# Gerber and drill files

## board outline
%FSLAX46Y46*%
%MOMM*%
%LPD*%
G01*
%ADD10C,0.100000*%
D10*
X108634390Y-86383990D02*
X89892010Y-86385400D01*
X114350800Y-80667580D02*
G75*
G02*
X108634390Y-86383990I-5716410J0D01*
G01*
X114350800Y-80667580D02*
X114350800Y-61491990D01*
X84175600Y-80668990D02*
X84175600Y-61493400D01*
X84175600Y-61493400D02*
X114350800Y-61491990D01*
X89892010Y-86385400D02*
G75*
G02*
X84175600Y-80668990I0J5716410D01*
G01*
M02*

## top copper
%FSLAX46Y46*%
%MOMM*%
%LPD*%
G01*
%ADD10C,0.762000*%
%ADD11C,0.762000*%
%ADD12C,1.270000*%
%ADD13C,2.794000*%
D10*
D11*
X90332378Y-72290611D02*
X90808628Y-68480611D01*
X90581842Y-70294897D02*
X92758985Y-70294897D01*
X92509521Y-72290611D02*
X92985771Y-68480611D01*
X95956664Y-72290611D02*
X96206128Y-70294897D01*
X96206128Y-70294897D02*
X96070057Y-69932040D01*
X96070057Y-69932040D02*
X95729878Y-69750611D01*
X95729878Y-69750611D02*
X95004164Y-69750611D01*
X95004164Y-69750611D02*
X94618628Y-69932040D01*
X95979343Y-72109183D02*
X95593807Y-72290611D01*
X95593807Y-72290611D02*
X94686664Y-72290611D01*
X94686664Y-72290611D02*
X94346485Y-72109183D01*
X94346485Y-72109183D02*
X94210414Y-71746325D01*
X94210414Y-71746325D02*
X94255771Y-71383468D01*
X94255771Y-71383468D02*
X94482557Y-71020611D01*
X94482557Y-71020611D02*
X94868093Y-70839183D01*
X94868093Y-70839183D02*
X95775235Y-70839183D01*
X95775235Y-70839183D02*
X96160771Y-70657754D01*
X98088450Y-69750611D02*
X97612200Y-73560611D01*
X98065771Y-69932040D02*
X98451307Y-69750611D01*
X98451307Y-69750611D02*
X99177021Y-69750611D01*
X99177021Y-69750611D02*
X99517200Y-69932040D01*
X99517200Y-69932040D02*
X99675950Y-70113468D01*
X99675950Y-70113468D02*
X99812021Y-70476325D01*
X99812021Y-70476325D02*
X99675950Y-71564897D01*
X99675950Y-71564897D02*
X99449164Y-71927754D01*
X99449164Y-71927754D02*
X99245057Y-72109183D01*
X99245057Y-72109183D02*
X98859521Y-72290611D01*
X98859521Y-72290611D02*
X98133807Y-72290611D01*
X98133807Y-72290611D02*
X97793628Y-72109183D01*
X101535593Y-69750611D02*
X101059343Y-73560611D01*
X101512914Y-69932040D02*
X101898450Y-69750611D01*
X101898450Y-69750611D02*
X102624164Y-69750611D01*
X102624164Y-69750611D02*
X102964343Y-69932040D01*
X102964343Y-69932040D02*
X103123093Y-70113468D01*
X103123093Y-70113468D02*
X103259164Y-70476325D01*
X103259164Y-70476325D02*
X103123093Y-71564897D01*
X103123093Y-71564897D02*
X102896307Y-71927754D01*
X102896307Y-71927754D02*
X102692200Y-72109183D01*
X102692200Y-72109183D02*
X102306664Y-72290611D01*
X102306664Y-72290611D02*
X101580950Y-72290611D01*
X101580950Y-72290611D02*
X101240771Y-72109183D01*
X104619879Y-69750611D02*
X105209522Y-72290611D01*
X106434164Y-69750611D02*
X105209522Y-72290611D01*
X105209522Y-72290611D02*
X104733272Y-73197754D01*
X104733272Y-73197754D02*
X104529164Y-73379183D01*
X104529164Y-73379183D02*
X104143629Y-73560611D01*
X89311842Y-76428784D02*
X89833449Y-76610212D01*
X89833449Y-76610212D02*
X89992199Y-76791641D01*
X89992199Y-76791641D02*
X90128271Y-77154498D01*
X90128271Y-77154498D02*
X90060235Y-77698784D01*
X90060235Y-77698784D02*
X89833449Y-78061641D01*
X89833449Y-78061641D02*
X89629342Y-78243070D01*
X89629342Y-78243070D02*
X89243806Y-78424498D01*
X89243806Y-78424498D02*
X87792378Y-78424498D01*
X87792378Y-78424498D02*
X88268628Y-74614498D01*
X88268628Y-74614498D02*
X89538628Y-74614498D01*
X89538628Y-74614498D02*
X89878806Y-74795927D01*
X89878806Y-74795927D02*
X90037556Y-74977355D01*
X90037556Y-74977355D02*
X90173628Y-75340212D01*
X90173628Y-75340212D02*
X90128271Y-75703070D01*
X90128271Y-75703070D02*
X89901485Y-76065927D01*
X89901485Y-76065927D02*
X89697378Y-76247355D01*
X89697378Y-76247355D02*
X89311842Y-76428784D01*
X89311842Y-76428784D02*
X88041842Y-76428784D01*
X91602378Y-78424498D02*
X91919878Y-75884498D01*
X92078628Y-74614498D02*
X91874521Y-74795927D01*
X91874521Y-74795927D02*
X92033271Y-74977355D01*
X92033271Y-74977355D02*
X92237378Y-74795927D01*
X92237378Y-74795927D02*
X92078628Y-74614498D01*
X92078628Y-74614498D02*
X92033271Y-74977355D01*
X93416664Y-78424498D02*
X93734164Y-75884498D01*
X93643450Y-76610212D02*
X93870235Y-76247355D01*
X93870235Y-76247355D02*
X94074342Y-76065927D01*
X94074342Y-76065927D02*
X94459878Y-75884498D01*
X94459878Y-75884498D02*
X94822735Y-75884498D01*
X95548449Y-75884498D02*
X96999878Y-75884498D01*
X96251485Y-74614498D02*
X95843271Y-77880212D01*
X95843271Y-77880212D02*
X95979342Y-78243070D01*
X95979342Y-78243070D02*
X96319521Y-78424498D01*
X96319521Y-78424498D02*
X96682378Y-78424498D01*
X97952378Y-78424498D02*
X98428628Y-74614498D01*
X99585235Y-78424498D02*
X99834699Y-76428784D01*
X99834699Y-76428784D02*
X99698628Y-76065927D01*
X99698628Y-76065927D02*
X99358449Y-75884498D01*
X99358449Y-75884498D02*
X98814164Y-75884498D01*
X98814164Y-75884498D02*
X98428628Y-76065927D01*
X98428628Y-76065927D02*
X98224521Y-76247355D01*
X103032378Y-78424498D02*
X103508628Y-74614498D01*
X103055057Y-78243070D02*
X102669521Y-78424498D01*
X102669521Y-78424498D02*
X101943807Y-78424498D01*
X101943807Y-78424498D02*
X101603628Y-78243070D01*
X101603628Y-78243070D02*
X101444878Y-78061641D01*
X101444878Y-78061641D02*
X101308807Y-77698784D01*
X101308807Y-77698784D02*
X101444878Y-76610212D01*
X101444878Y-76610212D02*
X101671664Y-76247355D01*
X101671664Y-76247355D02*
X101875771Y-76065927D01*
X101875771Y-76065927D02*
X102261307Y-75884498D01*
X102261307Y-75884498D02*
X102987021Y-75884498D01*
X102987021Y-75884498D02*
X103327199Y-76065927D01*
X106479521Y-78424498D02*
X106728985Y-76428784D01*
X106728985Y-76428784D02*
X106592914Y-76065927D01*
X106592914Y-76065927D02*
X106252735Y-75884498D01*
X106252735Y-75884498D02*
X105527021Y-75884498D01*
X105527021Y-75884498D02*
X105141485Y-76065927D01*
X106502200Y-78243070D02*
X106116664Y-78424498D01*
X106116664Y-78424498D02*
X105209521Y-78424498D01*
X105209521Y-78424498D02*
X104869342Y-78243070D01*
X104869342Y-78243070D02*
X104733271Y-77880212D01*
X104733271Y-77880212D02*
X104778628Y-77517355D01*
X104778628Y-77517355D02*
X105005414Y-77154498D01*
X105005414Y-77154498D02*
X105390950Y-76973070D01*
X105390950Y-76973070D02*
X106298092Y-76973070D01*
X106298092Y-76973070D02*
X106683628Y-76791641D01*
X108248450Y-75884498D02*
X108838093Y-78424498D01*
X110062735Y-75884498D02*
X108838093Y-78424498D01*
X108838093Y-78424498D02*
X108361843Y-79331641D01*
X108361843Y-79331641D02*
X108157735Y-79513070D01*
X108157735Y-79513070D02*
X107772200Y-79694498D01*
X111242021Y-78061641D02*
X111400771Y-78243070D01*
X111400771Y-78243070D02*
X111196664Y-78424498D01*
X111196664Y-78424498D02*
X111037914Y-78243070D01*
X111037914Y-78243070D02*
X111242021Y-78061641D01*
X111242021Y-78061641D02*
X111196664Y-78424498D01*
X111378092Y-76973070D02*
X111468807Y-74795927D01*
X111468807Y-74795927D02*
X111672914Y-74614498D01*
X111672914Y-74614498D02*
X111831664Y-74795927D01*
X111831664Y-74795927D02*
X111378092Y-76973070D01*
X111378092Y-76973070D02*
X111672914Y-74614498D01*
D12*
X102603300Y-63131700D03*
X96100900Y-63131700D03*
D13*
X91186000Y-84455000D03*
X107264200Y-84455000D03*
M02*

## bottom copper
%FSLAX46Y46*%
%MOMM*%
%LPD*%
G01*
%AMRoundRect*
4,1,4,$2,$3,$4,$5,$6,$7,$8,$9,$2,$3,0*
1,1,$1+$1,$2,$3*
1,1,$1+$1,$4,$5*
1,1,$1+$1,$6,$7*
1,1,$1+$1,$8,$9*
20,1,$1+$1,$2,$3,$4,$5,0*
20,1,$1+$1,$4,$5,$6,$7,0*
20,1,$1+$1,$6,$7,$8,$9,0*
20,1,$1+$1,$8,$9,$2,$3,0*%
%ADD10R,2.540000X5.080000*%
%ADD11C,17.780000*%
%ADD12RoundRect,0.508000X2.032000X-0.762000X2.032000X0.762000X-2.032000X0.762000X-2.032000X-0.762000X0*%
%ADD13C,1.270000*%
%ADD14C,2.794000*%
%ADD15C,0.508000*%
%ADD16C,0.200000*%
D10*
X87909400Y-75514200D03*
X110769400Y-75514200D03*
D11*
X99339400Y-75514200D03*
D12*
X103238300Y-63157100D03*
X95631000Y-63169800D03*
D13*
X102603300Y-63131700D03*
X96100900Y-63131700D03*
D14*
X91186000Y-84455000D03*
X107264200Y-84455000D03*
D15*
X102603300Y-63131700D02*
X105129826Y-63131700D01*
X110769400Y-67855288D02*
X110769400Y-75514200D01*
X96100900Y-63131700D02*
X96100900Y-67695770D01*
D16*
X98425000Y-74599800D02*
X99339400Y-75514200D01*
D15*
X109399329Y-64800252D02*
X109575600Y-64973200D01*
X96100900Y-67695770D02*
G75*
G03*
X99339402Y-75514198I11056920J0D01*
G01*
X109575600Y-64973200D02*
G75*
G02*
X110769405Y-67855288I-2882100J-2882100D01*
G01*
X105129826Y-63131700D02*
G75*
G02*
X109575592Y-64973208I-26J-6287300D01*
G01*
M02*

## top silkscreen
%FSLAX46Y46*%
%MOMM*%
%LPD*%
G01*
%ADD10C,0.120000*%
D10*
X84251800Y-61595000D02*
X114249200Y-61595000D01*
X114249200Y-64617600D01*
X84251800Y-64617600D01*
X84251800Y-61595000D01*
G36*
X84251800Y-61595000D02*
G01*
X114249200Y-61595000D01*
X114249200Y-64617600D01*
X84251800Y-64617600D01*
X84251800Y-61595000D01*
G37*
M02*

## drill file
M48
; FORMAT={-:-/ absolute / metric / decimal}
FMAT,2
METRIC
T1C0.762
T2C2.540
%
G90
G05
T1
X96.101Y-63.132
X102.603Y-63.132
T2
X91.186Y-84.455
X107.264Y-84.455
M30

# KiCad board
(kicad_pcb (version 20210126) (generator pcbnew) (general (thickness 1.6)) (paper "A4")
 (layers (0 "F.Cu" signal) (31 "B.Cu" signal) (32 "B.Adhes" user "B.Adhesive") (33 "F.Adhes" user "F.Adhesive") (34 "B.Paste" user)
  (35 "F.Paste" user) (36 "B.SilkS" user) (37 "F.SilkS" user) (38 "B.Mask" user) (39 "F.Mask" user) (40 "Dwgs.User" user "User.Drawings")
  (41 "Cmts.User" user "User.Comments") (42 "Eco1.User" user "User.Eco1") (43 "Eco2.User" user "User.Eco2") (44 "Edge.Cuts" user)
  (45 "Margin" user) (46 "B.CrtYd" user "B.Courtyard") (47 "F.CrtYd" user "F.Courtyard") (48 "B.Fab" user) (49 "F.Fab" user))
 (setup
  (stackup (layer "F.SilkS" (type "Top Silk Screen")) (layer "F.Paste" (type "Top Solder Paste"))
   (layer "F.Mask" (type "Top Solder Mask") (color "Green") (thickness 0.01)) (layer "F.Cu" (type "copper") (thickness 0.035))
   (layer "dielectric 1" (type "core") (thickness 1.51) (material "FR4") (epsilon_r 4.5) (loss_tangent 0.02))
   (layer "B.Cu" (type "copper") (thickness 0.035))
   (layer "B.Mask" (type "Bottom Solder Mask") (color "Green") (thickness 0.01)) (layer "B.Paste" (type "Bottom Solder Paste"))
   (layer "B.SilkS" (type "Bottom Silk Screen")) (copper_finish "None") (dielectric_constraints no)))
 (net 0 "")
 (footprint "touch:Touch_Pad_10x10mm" (layer "F.Cu") (at 102.3366 63.5762 -90)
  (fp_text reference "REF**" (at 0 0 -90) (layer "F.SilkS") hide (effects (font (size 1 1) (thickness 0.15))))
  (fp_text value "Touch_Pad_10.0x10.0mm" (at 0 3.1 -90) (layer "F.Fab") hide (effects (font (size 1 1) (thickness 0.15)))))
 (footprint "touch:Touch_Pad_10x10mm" (layer "F.Cu") (at 95.1865 63.5127 -90)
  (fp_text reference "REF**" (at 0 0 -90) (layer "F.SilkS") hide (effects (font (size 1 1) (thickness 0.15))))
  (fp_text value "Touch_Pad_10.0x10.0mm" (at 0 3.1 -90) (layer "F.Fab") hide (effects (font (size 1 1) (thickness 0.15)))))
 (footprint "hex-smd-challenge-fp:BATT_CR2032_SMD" (layer "B.Cu") (at 99.3394 75.5142 180)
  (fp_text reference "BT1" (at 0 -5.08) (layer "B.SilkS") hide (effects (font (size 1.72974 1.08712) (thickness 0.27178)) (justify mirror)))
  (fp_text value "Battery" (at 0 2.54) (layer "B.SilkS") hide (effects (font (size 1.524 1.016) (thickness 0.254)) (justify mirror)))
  (pad "1" smd rect (at 11.43 0 180) (locked) (size 2.54 5.08) (layers "B.Cu" "B.Paste" "B.Mask"))
  (pad "1" smd rect (at -11.43 0 180) (locked) (size 2.54 5.08) (layers "B.Cu" "B.Paste" "B.Mask"))
  (pad "2" smd circle (at 0 0 180) (locked) (size 17.78 17.78) (layers "B.Cu" "B.Paste" "B.Mask")))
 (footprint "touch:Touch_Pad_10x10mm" (layer "B.Cu") (at 101.7778 62.7888 90)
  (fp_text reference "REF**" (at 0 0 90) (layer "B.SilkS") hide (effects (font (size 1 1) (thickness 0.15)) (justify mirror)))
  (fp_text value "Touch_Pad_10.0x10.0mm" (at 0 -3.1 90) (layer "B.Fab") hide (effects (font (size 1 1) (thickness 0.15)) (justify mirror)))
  (pad "1" smd roundrect (at -0.3683 1.4605 90) (size 2.54 5.08) (layers "B.Cu" "B.Mask") (roundrect_rratio 0.2)))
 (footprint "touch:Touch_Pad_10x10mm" (layer "B.Cu") (at 95.1865 62.8523 90)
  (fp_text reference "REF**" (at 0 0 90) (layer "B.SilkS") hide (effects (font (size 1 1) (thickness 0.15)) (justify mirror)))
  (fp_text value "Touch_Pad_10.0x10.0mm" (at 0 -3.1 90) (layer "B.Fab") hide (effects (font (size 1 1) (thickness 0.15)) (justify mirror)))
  (pad "1" smd roundrect (at -0.3175 0.4445 90) (size 2.54 5.08) (layers "B.Cu" "B.Mask") (roundrect_rratio 0.2)))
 (gr_rect (start 84.2518 64.6176) (end 114.2492 61.595) (layer "F.SilkS") (width 0.12) (fill solid))
 (gr_line (start 108.63439 86.38399) (end 89.89201 86.3854) (layer "Edge.Cuts") (width 0.1))
 (gr_arc (start 108.63439 80.66758) (end 114.3508 80.66758) (angle 90) (layer "Edge.Cuts") (width 0.1))
 (gr_line (start 114.3508 80.66758) (end 114.3508 61.49199) (layer "Edge.Cuts") (width 0.1))
 (gr_line (start 84.1756 80.66899) (end 84.1756 61.4934) (layer "Edge.Cuts") (width 0.1))
 (gr_line (start 84.1756 61.4934) (end 114.3508 61.49199) (layer "Edge.Cuts") (width 0.1))
 (gr_arc (start 89.89201 80.66899) (end 84.1756 80.66899) (angle -90) (layer "Edge.Cuts") (width 0.1))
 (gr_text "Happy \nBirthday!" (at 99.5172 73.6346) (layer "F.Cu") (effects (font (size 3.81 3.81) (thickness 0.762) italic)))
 (via (at 102.6033 63.1317) (size 1.27) (drill 0.762) (layers "F.Cu" "B.Cu") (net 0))
 (via (at 96.1009 63.1317) (size 1.27) (drill 0.762) (layers "F.Cu" "B.Cu") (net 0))
 (via (at 91.186 84.455) (size 2.794) (drill 2.54) (layers "F.Cu" "B.Cu") (free) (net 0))
 (via (at 107.2642 84.455) (size 2.794) (drill 2.54) (layers "F.Cu" "B.Cu") (free) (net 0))
 (segment (start 102.6033 63.1317) (end 105.129826 63.1317) (width 0.508) (layer "B.Cu") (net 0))
 (segment (start 110.7694 67.855288) (end 110.7694 75.5142) (width 0.508) (layer "B.Cu") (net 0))
 (segment (start 96.1009 63.1317) (end 96.1009 67.69577) (width 0.508) (layer "B.Cu") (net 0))
 (segment (start 98.425 74.5998) (end 99.3394 75.5142) (width 0.2) (layer "B.Cu") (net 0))
 (segment (start 109.399329 64.800252) (end 109.5756 64.9732) (width 0.508) (layer "B.Cu") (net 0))
 (arc (start 96.1009 67.69577) (mid 96.942558 71.927073) (end 99.3394 75.5142) (width 0.508) (layer "B.Cu") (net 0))
 (arc (start 109.5756 64.9732) (mid 110.459141 66.295512) (end 110.7694 67.855288) (width 0.508) (layer "B.Cu") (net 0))
 (arc (start 105.129826 63.1317) (mid 107.535861 63.61029) (end 109.5756 64.9732) (width 0.508) (layer "B.Cu") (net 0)))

